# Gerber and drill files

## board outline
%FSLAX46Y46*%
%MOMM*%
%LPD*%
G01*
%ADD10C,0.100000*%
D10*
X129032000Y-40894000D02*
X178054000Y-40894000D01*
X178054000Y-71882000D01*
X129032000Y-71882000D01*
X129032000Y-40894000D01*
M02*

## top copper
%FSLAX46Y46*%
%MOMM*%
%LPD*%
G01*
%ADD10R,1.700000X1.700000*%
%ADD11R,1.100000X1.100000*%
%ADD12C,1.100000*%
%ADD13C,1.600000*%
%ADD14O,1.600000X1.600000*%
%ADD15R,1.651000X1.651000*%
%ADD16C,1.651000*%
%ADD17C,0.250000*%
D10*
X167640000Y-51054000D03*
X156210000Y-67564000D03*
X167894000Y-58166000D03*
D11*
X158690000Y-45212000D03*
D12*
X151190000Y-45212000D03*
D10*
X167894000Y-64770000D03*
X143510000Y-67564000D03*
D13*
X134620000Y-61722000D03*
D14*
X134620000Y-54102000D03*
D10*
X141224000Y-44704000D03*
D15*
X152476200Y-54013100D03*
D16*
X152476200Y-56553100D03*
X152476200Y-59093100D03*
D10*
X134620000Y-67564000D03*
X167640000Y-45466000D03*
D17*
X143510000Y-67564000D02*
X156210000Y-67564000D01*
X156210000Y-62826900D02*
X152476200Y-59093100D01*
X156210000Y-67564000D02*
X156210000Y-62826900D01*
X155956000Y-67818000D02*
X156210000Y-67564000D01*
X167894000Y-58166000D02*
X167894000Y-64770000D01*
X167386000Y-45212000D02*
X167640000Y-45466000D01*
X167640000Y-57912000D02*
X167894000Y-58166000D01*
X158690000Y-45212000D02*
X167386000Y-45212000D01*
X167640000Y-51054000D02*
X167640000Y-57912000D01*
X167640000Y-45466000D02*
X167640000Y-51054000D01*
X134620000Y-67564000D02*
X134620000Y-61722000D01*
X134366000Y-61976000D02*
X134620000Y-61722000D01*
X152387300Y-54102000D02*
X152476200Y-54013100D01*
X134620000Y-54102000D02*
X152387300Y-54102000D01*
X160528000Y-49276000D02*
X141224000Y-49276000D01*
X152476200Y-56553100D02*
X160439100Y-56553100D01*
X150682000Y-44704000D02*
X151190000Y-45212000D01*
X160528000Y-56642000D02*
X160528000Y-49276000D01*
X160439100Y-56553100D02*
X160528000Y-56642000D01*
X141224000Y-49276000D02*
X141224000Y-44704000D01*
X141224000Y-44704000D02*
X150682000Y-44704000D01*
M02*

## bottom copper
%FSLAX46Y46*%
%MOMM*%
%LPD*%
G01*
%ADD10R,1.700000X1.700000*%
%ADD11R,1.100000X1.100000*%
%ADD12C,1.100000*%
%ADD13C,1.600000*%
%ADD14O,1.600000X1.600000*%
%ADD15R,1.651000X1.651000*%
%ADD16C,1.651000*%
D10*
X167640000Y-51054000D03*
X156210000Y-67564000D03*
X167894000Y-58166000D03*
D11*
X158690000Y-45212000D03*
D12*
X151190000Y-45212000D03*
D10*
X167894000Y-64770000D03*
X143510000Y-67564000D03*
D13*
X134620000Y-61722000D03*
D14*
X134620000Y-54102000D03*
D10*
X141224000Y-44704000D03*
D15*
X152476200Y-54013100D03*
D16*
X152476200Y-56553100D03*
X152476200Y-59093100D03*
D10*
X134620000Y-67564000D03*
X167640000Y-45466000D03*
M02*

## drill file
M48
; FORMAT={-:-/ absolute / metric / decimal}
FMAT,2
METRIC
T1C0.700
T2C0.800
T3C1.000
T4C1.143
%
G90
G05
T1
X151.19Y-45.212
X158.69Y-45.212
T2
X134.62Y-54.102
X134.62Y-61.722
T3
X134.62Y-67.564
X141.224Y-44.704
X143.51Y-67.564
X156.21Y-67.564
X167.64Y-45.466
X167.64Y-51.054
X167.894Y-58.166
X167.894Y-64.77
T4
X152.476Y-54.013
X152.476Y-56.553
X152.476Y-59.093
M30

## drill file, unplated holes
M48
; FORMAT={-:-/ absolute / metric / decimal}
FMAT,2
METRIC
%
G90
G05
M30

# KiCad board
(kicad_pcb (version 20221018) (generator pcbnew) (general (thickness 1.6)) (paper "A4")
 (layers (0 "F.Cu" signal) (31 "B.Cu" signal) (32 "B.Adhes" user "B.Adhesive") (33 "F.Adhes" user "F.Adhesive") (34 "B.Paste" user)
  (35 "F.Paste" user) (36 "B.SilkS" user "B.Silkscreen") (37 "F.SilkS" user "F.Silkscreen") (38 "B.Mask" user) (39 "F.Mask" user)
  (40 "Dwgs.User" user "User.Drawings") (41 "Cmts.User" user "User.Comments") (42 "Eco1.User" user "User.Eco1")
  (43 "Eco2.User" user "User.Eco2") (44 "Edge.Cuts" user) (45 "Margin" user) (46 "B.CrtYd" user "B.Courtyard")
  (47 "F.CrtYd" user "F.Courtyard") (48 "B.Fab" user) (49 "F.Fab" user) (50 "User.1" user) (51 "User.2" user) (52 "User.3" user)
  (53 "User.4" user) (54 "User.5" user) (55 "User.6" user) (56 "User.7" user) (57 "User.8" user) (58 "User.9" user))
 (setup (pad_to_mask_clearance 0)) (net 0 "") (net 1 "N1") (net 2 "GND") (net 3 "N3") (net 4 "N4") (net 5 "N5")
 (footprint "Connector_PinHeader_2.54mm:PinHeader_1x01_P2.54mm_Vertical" (layer "F.Cu") (at 167.64 51.054)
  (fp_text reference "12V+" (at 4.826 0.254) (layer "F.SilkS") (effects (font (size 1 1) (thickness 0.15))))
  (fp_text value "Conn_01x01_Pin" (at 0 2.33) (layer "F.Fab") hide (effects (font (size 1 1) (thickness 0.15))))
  (pad "1" thru_hole rect (at 0 0) (size 1.7 1.7) (drill 1) (layers "*.Cu" "*.Mask") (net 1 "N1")))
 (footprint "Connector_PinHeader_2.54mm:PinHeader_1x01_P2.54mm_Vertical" (layer "F.Cu") (at 156.21 67.564)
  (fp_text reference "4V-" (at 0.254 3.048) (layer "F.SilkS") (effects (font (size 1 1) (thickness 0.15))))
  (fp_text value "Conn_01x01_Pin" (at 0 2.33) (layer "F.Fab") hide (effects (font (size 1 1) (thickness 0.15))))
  (pad "1" thru_hole rect (at 0 0) (size 1.7 1.7) (drill 1) (layers "*.Cu" "*.Mask") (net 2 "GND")))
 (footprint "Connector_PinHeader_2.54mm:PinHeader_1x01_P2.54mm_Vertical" (layer "F.Cu") (at 167.894 58.166)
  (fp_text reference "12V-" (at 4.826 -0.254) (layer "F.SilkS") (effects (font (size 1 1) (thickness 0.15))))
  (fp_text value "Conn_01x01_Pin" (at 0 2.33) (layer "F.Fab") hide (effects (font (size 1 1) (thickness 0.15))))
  (pad "1" thru_hole rect (at 0 0) (size 1.7 1.7) (drill 1) (layers "*.Cu" "*.Mask") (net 1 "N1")))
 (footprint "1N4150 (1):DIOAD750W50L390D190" (layer "F.Cu") (at 154.94 45.212 180)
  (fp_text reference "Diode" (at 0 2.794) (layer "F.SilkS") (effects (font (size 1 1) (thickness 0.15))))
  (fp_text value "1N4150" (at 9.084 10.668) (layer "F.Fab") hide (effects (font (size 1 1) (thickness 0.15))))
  (pad "1" thru_hole rect (at -3.75 0 180) (size 1.1 1.1) (drill 0.7) (layers "*.Cu" "*.Mask") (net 1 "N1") (solder_mask_margin 0.102))
  (pad "2" thru_hole circle (at 3.75 0 180) (size 1.1 1.1) (drill 0.7) (layers "*.Cu" "*.Mask") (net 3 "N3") (solder_mask_margin 0.102)))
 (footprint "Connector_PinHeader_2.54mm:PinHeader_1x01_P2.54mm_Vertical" (layer "F.Cu") (at 167.894 64.77)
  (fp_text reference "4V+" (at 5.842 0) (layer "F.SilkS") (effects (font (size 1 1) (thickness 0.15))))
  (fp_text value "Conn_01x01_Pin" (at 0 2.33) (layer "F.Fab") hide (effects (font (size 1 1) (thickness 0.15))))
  (pad "1" thru_hole rect (at 0 0) (size 1.7 1.7) (drill 1) (layers "*.Cu" "*.Mask") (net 1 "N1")))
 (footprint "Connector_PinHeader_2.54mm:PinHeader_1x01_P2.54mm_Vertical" (layer "F.Cu") (at 143.51 67.564)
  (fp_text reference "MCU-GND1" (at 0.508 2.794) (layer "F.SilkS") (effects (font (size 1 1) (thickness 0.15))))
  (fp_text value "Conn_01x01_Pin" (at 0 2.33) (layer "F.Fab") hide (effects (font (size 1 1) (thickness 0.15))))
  (pad "1" thru_hole rect (at 0 0) (size 1.7 1.7) (drill 1) (layers "*.Cu" "*.Mask") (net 2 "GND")))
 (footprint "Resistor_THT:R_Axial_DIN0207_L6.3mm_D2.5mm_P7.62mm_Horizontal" (layer "F.Cu") (at 134.62 61.722 90)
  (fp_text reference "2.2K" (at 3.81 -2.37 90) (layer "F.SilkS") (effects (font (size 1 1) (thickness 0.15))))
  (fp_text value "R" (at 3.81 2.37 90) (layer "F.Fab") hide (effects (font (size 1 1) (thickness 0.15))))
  (pad "1" thru_hole circle (at 0 0 90) (size 1.6 1.6) (drill 0.8) (layers "*.Cu" "*.Mask") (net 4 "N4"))
  (pad "2" thru_hole oval (at 7.62 0 90) (size 1.6 1.6) (drill 0.8) (layers "*.Cu" "*.Mask") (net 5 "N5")))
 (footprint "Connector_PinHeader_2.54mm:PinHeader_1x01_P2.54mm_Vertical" (layer "F.Cu") (at 141.224 44.704)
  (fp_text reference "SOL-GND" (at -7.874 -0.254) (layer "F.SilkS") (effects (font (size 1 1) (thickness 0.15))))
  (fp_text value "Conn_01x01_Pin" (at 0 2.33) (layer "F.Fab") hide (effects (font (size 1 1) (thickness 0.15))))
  (pad "1" thru_hole rect (at 0 0) (size 1.7 1.7) (drill 1) (layers "*.Cu" "*.Mask") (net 3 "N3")))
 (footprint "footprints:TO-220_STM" (layer "F.Cu") (at 152.4762 54.0131 -90)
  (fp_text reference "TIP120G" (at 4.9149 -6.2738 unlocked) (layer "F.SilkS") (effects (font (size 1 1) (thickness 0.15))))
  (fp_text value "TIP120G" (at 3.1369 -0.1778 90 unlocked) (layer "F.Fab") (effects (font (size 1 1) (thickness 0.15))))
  (pad "1" thru_hole rect (at 0 0 270) (size 1.651 1.651) (drill 1.143) (layers "*.Cu" "*.Mask") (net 5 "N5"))
  (pad "2" thru_hole circle (at 2.54 0 270) (size 1.651 1.651) (drill 1.143) (layers "*.Cu" "*.Mask") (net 3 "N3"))
  (pad "3" thru_hole circle (at 5.08 0 270) (size 1.651 1.651) (drill 1.143) (layers "*.Cu" "*.Mask") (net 2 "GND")))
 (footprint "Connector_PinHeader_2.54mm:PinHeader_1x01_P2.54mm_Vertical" (layer "F.Cu") (at 134.62 67.564 90)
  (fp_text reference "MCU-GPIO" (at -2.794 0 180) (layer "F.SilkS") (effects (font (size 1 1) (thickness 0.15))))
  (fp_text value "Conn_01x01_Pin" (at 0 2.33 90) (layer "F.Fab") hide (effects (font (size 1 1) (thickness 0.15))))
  (pad "1" thru_hole rect (at 0 0 90) (size 1.7 1.7) (drill 1) (layers "*.Cu" "*.Mask") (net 4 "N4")))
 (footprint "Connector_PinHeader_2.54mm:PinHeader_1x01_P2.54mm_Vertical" (layer "F.Cu") (at 167.64 45.466)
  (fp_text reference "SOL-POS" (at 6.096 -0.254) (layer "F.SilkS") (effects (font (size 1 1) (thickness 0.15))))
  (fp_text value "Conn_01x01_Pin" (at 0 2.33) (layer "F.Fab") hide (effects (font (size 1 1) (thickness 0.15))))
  (pad "1" thru_hole rect (at 0 0) (size 1.7 1.7) (drill 1) (layers "*.Cu" "*.Mask") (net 1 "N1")))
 (gr_rect (start 129.032 40.894) (end 178.054 71.882) (stroke (width 0.1) (type default)) (fill none) (layer "Edge.Cuts"))
 (segment (start 143.51 67.564) (end 156.21 67.564) (width 0.25) (layer "F.Cu") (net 2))
 (segment (start 156.21 62.8269) (end 152.4762 59.0931) (width 0.25) (layer "F.Cu") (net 2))
 (segment (start 156.21 67.564) (end 156.21 62.8269) (width 0.25) (layer "F.Cu") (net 2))
 (segment (start 155.956 67.818) (end 156.21 67.564) (width 0.25) (layer "F.Cu") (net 2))
 (segment (start 167.894 58.166) (end 167.894 64.77) (width 0.25) (layer "F.Cu") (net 1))
 (segment (start 167.386 45.212) (end 167.64 45.466) (width 0.25) (layer "F.Cu") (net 1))
 (segment (start 167.64 57.912) (end 167.894 58.166) (width 0.25) (layer "F.Cu") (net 1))
 (segment (start 158.69 45.212) (end 167.386 45.212) (width 0.25) (layer "F.Cu") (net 1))
 (segment (start 167.64 51.054) (end 167.64 57.912) (width 0.25) (layer "F.Cu") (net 1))
 (segment (start 167.64 45.466) (end 167.64 51.054) (width 0.25) (layer "F.Cu") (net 1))
 (segment (start 134.62 67.564) (end 134.62 61.722) (width 0.25) (layer "F.Cu") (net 4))
 (segment (start 134.366 61.976) (end 134.62 61.722) (width 0.25) (layer "F.Cu") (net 4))
 (segment (start 152.3873 54.102) (end 152.4762 54.0131) (width 0.25) (layer "F.Cu") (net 5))
 (segment (start 134.62 54.102) (end 152.3873 54.102) (width 0.25) (layer "F.Cu") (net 5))
 (segment (start 160.528 49.276) (end 141.224 49.276) (width 0.25) (layer "F.Cu") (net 3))
 (segment (start 152.4762 56.5531) (end 160.4391 56.5531) (width 0.25) (layer "F.Cu") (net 3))
 (segment (start 150.682 44.704) (end 151.19 45.212) (width 0.25) (layer "F.Cu") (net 3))
 (segment (start 160.528 56.642) (end 160.528 49.276) (width 0.25) (layer "F.Cu") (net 3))
 (segment (start 160.4391 56.5531) (end 160.528 56.642) (width 0.25) (layer "F.Cu") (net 3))
 (segment (start 141.224 49.276) (end 141.224 44.704) (width 0.25) (layer "F.Cu") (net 3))
 (segment (start 141.224 44.704) (end 150.682 44.704) (width 0.25) (layer "F.Cu") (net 3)))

